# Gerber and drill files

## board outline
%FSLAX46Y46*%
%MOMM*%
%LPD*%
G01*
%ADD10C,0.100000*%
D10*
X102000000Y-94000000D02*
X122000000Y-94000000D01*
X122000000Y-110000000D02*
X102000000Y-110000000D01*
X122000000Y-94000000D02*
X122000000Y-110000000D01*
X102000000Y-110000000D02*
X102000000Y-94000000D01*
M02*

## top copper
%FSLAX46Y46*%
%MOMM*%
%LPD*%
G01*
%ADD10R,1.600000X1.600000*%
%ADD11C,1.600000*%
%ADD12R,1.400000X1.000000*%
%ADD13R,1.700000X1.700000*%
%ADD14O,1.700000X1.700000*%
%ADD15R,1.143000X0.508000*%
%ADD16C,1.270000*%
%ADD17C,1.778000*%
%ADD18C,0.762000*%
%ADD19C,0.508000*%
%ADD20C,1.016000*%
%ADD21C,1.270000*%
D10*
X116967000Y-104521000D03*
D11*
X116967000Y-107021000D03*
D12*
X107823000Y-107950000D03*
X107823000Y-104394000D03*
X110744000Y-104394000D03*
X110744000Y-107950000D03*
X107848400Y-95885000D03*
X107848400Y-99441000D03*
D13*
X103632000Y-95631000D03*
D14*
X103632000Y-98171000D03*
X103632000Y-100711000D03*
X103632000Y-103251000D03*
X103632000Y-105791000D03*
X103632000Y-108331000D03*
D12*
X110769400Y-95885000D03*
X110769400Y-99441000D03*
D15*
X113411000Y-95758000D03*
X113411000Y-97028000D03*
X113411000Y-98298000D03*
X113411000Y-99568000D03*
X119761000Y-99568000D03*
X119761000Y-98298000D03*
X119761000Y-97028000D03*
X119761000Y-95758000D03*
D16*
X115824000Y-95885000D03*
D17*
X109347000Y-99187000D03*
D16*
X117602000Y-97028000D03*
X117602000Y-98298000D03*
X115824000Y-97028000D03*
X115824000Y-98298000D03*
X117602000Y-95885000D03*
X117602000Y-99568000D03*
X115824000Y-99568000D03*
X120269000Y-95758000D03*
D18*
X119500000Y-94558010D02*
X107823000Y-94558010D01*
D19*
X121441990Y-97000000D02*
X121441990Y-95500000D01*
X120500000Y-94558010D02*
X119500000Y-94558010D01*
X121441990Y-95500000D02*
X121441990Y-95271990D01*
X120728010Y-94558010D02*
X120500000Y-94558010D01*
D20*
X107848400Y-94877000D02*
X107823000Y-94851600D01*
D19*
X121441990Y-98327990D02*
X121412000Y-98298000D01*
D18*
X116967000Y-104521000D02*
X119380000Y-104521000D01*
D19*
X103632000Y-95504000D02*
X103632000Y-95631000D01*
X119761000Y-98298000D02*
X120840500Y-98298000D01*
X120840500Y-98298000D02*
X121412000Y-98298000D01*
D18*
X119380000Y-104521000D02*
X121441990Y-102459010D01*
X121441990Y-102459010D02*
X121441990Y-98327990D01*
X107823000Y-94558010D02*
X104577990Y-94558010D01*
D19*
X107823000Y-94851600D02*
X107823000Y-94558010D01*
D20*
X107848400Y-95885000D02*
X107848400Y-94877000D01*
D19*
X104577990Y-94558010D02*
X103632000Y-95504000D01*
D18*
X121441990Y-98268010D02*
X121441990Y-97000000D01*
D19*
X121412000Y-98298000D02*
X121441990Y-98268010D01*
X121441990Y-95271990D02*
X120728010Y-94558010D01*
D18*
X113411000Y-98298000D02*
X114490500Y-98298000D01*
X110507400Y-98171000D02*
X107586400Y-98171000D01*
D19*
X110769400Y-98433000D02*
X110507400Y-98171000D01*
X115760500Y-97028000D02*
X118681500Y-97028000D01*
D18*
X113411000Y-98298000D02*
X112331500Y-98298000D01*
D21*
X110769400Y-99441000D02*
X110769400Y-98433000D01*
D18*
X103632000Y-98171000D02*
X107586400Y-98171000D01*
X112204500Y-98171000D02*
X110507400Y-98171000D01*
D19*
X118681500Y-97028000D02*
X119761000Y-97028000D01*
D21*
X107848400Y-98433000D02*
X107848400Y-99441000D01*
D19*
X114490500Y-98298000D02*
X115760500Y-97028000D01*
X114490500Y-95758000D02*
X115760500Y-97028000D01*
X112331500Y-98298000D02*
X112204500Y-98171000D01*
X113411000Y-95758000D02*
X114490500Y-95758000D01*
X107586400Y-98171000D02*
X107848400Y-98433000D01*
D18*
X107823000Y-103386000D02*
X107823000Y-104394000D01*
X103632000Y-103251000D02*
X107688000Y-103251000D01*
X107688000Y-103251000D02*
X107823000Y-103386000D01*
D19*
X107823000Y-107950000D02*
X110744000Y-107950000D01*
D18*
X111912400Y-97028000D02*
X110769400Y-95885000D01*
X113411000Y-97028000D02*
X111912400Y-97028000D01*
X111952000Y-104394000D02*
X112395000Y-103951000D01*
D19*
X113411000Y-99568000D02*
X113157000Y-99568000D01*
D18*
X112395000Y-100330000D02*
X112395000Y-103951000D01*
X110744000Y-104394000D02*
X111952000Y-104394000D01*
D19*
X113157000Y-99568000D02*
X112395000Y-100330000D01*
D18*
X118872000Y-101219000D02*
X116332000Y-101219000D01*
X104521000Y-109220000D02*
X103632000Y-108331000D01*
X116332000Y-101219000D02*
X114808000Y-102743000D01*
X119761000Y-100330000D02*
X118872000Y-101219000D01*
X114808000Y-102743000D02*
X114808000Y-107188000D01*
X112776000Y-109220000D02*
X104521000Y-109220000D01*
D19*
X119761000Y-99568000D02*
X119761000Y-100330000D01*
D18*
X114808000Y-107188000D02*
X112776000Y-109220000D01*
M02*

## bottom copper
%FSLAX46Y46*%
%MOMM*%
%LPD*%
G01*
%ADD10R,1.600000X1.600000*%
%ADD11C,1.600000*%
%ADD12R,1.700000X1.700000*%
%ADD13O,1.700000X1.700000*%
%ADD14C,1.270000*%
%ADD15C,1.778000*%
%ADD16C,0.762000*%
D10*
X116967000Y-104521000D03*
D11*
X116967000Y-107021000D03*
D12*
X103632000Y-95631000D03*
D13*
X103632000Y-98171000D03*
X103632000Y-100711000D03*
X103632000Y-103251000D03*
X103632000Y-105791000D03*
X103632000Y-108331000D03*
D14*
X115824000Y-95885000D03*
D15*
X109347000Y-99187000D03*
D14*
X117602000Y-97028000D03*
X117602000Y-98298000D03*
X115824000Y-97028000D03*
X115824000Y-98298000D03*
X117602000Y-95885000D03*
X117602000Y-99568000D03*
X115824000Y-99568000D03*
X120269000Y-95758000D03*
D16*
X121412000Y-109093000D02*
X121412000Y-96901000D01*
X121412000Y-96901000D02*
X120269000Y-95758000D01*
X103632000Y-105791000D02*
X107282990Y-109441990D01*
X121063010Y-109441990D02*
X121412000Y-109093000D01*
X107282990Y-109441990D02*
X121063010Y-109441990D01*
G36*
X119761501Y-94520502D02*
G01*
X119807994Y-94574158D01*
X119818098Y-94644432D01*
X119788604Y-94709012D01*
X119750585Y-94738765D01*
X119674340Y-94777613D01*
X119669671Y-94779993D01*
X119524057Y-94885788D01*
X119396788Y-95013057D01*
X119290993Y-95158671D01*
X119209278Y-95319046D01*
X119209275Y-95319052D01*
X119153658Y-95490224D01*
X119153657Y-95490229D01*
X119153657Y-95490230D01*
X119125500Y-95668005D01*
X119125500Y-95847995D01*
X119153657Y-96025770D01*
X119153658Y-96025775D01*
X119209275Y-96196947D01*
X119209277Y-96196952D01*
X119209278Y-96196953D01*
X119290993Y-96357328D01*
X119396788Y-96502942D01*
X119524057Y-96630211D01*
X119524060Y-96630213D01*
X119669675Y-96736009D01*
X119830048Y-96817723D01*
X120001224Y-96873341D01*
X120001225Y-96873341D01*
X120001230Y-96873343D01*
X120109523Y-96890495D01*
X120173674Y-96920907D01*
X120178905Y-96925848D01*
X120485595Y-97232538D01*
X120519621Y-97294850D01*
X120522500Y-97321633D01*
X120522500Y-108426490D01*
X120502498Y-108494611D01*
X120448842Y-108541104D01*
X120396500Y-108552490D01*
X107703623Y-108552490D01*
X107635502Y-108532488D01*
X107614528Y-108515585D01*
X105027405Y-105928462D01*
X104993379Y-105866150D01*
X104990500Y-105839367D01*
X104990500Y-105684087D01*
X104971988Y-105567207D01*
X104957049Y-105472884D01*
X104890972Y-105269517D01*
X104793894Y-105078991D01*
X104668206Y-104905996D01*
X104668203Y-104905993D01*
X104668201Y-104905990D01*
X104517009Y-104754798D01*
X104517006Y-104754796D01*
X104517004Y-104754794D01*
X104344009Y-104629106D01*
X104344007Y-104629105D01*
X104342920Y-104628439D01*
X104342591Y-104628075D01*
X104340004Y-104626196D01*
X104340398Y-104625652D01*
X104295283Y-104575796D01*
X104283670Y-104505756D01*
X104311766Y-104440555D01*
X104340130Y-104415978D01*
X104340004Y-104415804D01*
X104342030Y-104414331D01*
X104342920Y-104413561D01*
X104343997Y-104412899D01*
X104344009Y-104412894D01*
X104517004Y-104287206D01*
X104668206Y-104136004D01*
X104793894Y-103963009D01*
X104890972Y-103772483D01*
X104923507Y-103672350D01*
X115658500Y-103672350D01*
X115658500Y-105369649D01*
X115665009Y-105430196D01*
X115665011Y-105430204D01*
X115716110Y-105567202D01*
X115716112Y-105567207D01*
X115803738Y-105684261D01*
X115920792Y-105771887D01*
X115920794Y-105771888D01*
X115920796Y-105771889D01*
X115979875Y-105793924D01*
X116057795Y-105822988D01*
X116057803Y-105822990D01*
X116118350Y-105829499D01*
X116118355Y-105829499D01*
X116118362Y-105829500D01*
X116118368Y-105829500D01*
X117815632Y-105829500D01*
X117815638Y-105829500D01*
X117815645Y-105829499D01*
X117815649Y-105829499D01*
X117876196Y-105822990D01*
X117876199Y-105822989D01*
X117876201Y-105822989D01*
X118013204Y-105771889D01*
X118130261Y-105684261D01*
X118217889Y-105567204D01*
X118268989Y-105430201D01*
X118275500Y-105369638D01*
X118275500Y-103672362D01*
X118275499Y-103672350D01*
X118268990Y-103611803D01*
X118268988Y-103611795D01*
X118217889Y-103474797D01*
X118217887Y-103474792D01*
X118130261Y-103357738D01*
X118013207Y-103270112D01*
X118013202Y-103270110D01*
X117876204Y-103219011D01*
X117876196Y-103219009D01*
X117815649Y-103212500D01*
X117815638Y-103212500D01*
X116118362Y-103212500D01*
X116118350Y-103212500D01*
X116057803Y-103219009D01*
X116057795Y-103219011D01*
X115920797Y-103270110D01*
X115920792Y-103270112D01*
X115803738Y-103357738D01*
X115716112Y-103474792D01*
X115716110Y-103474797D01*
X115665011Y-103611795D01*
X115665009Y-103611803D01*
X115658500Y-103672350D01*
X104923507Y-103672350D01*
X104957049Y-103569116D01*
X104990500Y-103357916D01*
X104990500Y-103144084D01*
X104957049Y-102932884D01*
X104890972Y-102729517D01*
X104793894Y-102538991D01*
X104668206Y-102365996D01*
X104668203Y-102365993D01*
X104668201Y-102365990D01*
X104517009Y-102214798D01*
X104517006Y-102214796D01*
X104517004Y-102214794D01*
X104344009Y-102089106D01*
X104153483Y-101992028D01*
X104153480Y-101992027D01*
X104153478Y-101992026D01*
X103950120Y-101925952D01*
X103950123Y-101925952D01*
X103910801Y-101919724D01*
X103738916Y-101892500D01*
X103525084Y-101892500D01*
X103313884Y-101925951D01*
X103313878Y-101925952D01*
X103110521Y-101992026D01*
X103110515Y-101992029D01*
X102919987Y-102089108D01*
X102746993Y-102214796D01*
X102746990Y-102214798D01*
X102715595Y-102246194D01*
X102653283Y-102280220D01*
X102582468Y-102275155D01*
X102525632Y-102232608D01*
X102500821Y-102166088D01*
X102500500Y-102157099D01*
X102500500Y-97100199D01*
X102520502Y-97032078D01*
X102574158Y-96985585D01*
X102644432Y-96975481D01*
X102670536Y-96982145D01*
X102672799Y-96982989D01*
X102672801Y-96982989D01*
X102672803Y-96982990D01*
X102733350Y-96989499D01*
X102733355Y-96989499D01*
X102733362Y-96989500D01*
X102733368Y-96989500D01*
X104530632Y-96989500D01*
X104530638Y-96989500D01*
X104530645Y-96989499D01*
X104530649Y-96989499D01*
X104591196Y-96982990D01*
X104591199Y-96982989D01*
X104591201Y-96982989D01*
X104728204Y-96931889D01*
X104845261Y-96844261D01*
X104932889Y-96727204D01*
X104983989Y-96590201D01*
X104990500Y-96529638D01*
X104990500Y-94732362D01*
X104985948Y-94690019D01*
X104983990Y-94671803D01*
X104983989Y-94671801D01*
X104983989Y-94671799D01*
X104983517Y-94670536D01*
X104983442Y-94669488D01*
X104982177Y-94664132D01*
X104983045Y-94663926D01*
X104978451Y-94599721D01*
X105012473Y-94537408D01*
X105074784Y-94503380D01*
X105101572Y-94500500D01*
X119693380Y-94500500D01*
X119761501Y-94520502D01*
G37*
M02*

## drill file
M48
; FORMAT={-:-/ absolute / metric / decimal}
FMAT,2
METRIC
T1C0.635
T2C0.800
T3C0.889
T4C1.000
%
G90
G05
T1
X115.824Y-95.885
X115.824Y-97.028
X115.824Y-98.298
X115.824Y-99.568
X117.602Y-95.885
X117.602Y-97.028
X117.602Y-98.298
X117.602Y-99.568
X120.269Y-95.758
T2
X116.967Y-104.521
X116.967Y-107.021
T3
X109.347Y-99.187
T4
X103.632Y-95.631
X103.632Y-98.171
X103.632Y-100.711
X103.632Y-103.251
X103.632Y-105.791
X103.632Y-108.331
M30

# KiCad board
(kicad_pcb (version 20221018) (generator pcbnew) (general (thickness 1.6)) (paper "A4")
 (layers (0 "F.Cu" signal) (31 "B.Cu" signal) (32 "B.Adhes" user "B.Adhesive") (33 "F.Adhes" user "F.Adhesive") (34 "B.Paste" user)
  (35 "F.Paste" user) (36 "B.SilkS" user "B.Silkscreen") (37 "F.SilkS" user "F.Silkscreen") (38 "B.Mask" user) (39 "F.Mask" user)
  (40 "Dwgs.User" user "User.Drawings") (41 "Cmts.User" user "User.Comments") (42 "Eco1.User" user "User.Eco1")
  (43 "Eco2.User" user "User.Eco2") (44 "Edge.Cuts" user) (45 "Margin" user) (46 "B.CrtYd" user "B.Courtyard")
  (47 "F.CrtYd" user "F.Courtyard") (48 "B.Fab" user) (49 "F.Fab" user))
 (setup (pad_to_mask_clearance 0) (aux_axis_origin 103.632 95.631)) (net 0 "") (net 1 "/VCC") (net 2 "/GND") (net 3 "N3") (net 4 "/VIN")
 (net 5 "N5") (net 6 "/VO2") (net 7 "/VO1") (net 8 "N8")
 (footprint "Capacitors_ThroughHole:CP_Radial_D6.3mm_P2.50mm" (layer "F.Cu") (at 116.967 104.521 -90)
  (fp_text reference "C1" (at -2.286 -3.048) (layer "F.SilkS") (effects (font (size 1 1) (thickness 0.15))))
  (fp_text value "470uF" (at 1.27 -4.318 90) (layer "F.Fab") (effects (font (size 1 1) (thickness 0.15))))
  (pad "1" thru_hole rect (at 0 0 270) (size 1.6 1.6) (drill 0.8) (layers "*.Cu" "*.Mask") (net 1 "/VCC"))
  (pad "2" thru_hole circle (at 2.5 0 270) (size 1.6 1.6) (drill 0.8) (layers "*.Cu" "*.Mask") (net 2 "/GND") (zone_connect 2)))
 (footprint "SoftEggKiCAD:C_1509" (layer "F.Cu") (at 107.9754 106.426 90)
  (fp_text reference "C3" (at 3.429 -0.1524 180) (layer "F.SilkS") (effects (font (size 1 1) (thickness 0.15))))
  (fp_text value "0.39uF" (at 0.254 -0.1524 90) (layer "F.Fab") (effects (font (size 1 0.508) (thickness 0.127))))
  (pad "1" smd rect (at -1.524 -0.1524 90) (size 1 1.4) (layers "F.Cu" "F.Paste" "F.Mask") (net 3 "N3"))
  (pad "2" smd rect (at 2.032 -0.1524 90) (size 1 1.4) (layers "F.Cu" "F.Paste" "F.Mask") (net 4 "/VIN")))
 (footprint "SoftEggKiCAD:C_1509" (layer "F.Cu") (at 110.5916 105.918 -90)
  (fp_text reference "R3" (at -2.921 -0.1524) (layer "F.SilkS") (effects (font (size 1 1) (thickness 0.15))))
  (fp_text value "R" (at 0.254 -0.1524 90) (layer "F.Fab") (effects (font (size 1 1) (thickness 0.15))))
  (pad "1" smd rect (at -1.524 -0.1524 270) (size 1 1.4) (layers "F.Cu" "F.Paste" "F.Mask") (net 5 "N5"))
  (pad "2" smd rect (at 2.032 -0.1524 270) (size 1 1.4) (layers "F.Cu" "F.Paste" "F.Mask") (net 3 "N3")))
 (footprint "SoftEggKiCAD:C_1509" (layer "F.Cu") (at 107.696 97.409 -90)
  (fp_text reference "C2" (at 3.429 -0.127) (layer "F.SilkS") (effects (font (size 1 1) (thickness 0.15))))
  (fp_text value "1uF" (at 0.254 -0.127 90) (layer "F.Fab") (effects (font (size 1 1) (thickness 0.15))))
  (pad "1" smd rect (at -1.524 -0.1524 270) (size 1 1.4) (layers "F.Cu" "F.Paste" "F.Mask") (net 1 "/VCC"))
  (pad "2" smd rect (at 2.032 -0.1524 270) (size 1 1.4) (layers "F.Cu" "F.Paste" "F.Mask") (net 2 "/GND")))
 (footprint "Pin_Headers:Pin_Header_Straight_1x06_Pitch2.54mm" (layer "F.Cu") (at 103.632 95.631)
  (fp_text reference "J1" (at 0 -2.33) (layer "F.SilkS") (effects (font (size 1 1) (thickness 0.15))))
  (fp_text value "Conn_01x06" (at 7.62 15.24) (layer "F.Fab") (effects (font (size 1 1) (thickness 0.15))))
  (pad "1" thru_hole rect (at 0 0) (size 1.7 1.7) (drill 1) (layers "*.Cu" "*.Mask") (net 1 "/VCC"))
  (pad "2" thru_hole oval (at 0 2.54) (size 1.7 1.7) (drill 1) (layers "*.Cu" "*.Mask") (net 2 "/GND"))
  (pad "3" thru_hole oval (at 0 5.08) (size 1.7 1.7) (drill 1) (layers "*.Cu" "*.Mask") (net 2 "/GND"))
  (pad "4" thru_hole oval (at 0 7.62) (size 1.7 1.7) (drill 1) (layers "*.Cu" "*.Mask") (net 4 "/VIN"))
  (pad "5" thru_hole oval (at 0 10.16) (size 1.7 1.7) (drill 1) (layers "*.Cu" "*.Mask") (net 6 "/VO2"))
  (pad "6" thru_hole oval (at 0 12.7) (size 1.7 1.7) (drill 1) (layers "*.Cu" "*.Mask") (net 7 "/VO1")))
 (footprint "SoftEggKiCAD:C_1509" (layer "F.Cu") (at 110.617 97.409 -90)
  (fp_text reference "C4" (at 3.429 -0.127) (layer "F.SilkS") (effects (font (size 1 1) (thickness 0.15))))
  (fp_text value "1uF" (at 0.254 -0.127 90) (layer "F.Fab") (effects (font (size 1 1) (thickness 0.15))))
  (pad "1" smd rect (at -1.524 -0.1524 270) (size 1 1.4) (layers "F.Cu" "F.Paste" "F.Mask") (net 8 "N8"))
  (pad "2" smd rect (at 2.032 -0.1524 270) (size 1 1.4) (layers "F.Cu" "F.Paste" "F.Mask") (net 2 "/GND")))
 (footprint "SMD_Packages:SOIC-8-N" (layer "F.Cu") (at 116.586 97.663 -90)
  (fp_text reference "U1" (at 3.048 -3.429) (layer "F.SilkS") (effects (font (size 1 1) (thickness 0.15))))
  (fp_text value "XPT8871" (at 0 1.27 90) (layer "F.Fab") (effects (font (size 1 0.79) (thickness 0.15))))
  (pad "1" smd rect (at -1.905 3.175 270) (size 0.508 1.143) (layers "F.Cu" "F.Paste" "F.Mask") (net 2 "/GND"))
  (pad "2" smd rect (at -0.635 3.175 270) (size 0.508 1.143) (layers "F.Cu" "F.Paste" "F.Mask") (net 8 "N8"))
  (pad "3" smd rect (at 0.635 3.175 270) (size 0.508 1.143) (layers "F.Cu" "F.Paste" "F.Mask") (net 2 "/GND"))
  (pad "4" smd rect (at 1.905 3.175 270) (size 0.508 1.143) (layers "F.Cu" "F.Paste" "F.Mask") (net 5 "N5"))
  (pad "5" smd rect (at 1.905 -3.175 270) (size 0.508 1.143) (layers "F.Cu" "F.Paste" "F.Mask") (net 7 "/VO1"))
  (pad "6" smd rect (at 0.635 -3.175 270) (size 0.508 1.143) (layers "F.Cu" "F.Paste" "F.Mask") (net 1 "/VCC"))
  (pad "7" smd rect (at -0.635 -3.175 270) (size 0.508 1.143) (layers "F.Cu" "F.Paste" "F.Mask") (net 2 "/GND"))
  (pad "8" smd rect (at -1.905 -3.175 270) (size 0.508 1.143) (layers "F.Cu" "F.Paste" "F.Mask") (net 6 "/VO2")))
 (gr_line (start 102 94) (end 122 94) (stroke (width 0.1) (type solid)) (layer "Edge.Cuts"))
 (gr_line (start 122 110) (end 102 110) (stroke (width 0.1) (type solid)) (layer "Edge.Cuts"))
 (gr_line (start 122 94) (end 122 110) (stroke (width 0.1) (type solid)) (layer "Edge.Cuts"))
 (gr_line (start 102 110) (end 102 94) (stroke (width 0.1) (type solid)) (layer "Edge.Cuts"))
 (segment (start 119.5 94.55801) (end 107.823 94.55801) (width 0.762) (layer "F.Cu") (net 1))
 (segment (start 121.44199 97) (end 121.44199 95.5) (width 0.508) (layer "F.Cu") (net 1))
 (segment (start 120.5 94.55801) (end 119.5 94.55801) (width 0.508) (layer "F.Cu") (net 1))
 (segment (start 121.44199 95.5) (end 121.44199 95.27199) (width 0.508) (layer "F.Cu") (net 1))
 (segment (start 120.72801 94.55801) (end 120.5 94.55801) (width 0.508) (layer "F.Cu") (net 1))
 (segment (start 107.8484 94.877) (end 107.823 94.8516) (width 1.016) (layer "F.Cu") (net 1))
 (segment (start 121.44199 98.32799) (end 121.412 98.298) (width 0.508) (layer "F.Cu") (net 1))
 (segment (start 116.967 104.521) (end 119.38 104.521) (width 0.762) (layer "F.Cu") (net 1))
 (segment (start 103.632 95.504) (end 103.632 95.631) (width 0.508) (layer "F.Cu") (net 1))
 (segment (start 119.761 98.298) (end 120.8405 98.298) (width 0.508) (layer "F.Cu") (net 1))
 (segment (start 120.8405 98.298) (end 121.412 98.298) (width 0.508) (layer "F.Cu") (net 1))
 (segment (start 119.38 104.521) (end 121.44199 102.45901) (width 0.762) (layer "F.Cu") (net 1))
 (segment (start 121.44199 102.45901) (end 121.44199 98.32799) (width 0.762) (layer "F.Cu") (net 1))
 (segment (start 107.823 94.55801) (end 104.57799 94.55801) (width 0.762) (layer "F.Cu") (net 1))
 (segment (start 107.823 94.8516) (end 107.823 94.55801) (width 0.508) (layer "F.Cu") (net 1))
 (segment (start 107.8484 95.885) (end 107.8484 94.877) (width 1.016) (layer "F.Cu") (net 1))
 (segment (start 104.57799 94.55801) (end 103.632 95.504) (width 0.508) (layer "F.Cu") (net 1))
 (segment (start 121.44199 98.26801) (end 121.44199 97) (width 0.762) (layer "F.Cu") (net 1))
 (segment (start 121.412 98.298) (end 121.44199 98.26801) (width 0.508) (layer "F.Cu") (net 1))
 (segment (start 121.44199 95.27199) (end 120.72801 94.55801) (width 0.508) (layer "F.Cu") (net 1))
 (segment (start 113.411 98.298) (end 114.4905 98.298) (width 0.762) (layer "F.Cu") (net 2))
 (segment (start 110.5074 98.171) (end 107.5864 98.171) (width 0.762) (layer "F.Cu") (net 2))
 (segment (start 110.7694 98.433) (end 110.5074 98.171) (width 0.508) (layer "F.Cu") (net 2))
 (segment (start 115.7605 97.028) (end 118.6815 97.028) (width 0.508) (layer "F.Cu") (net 2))
 (segment (start 113.411 98.298) (end 112.3315 98.298) (width 0.762) (layer "F.Cu") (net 2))
 (segment (start 110.7694 99.441) (end 110.7694 98.433) (width 1.27) (layer "F.Cu") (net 2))
 (segment (start 103.632 98.171) (end 107.5864 98.171) (width 0.762) (layer "F.Cu") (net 2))
 (segment (start 112.2045 98.171) (end 110.5074 98.171) (width 0.762) (layer "F.Cu") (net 2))
 (segment (start 118.6815 97.028) (end 119.761 97.028) (width 0.508) (layer "F.Cu") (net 2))
 (segment (start 107.8484 98.433) (end 107.8484 99.441) (width 1.27) (layer "F.Cu") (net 2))
 (segment (start 114.4905 98.298) (end 115.7605 97.028) (width 0.508) (layer "F.Cu") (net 2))
 (segment (start 114.4905 95.758) (end 115.7605 97.028) (width 0.508) (layer "F.Cu") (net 2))
 (segment (start 112.3315 98.298) (end 112.2045 98.171) (width 0.508) (layer "F.Cu") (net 2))
 (segment (start 113.411 95.758) (end 114.4905 95.758) (width 0.508) (layer "F.Cu") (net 2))
 (segment (start 107.5864 98.171) (end 107.8484 98.433) (width 0.508) (layer "F.Cu") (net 2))
 (via (at 115.824 95.885) (size 1.27) (drill 0.635) (layers "F.Cu" "B.Cu") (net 2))
 (via (at 109.347 99.187) (size 1.778) (drill 0.889) (layers "F.Cu" "B.Cu") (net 2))
 (via (at 117.602 97.028) (size 1.27) (drill 0.635) (layers "F.Cu" "B.Cu") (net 2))
 (via (at 117.602 98.298) (size 1.27) (drill 0.635) (layers "F.Cu" "B.Cu") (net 2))
 (via (at 115.824 97.028) (size 1.27) (drill 0.635) (layers "F.Cu" "B.Cu") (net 2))
 (via (at 115.824 98.298) (size 1.27) (drill 0.635) (layers "F.Cu" "B.Cu") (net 2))
 (via (at 117.602 95.885) (size 1.27) (drill 0.635) (layers "F.Cu" "B.Cu") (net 2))
 (via (at 117.602 99.568) (size 1.27) (drill 0.635) (layers "F.Cu" "B.Cu") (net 2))
 (via (at 115.824 99.568) (size 1.27) (drill 0.635) (layers "F.Cu" "B.Cu") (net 2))
 (segment (start 107.823 103.386) (end 107.823 104.394) (width 0.762) (layer "F.Cu") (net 4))
 (segment (start 103.632 103.251) (end 107.688 103.251) (width 0.762) (layer "F.Cu") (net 4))
 (segment (start 107.688 103.251) (end 107.823 103.386) (width 0.762) (layer "F.Cu") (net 4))
 (segment (start 107.823 107.95) (end 110.744 107.95) (width 0.508) (layer "F.Cu") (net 3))
 (segment (start 111.9124 97.028) (end 110.7694 95.885) (width 0.762) (layer "F.Cu") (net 8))
 (segment (start 113.411 97.028) (end 111.9124 97.028) (width 0.762) (layer "F.Cu") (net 8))
 (segment (start 111.952 104.394) (end 112.395 103.951) (width 0.762) (layer "F.Cu") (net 5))
 (segment (start 113.411 99.568) (end 113.157 99.568) (width 0.508) (layer "F.Cu") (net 5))
 (segment (start 112.395 100.33) (end 112.395 103.951) (width 0.762) (layer "F.Cu") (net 5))
 (segment (start 110.744 104.394) (end 111.952 104.394) (width 0.762) (layer "F.Cu") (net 5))
 (segment (start 113.157 99.568) (end 112.395 100.33) (width 0.508) (layer "F.Cu") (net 5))
 (segment (start 118.872 101.219) (end 116.332 101.219) (width 0.762) (layer "F.Cu") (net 7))
 (segment (start 104.521 109.22) (end 103.632 108.331) (width 0.762) (layer "F.Cu") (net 7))
 (segment (start 116.332 101.219) (end 114.808 102.743) (width 0.762) (layer "F.Cu") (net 7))
 (segment (start 119.761 100.33) (end 118.872 101.219) (width 0.762) (layer "F.Cu") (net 7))
 (segment (start 114.808 102.743) (end 114.808 107.188) (width 0.762) (layer "F.Cu") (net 7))
 (segment (start 112.776 109.22) (end 104.521 109.22) (width 0.762) (layer "F.Cu") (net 7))
 (segment (start 119.761 99.568) (end 119.761 100.33) (width 0.508) (layer "F.Cu") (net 7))
 (segment (start 114.808 107.188) (end 112.776 109.22) (width 0.762) (layer "F.Cu") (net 7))
 (via (at 120.269 95.758) (size 1.27) (drill 0.635) (layers "F.Cu" "B.Cu") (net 6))
 (segment (start 121.412 109.093) (end 121.412 96.901) (width 0.762) (layer "B.Cu") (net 6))
 (segment (start 121.412 96.901) (end 120.269 95.758) (width 0.762) (layer "B.Cu") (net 6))
 (segment (start 103.632 105.791) (end 107.28299 109.44199) (width 0.762) (layer "B.Cu") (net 6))
 (segment (start 121.06301 109.44199) (end 121.412 109.093) (width 0.762) (layer "B.Cu") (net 6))
 (segment (start 107.28299 109.44199) (end 121.06301 109.44199) (width 0.762) (layer "B.Cu") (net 6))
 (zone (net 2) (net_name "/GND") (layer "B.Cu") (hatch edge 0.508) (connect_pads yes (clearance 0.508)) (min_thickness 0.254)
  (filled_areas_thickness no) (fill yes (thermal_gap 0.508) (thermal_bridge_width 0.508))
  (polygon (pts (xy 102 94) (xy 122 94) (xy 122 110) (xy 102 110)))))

